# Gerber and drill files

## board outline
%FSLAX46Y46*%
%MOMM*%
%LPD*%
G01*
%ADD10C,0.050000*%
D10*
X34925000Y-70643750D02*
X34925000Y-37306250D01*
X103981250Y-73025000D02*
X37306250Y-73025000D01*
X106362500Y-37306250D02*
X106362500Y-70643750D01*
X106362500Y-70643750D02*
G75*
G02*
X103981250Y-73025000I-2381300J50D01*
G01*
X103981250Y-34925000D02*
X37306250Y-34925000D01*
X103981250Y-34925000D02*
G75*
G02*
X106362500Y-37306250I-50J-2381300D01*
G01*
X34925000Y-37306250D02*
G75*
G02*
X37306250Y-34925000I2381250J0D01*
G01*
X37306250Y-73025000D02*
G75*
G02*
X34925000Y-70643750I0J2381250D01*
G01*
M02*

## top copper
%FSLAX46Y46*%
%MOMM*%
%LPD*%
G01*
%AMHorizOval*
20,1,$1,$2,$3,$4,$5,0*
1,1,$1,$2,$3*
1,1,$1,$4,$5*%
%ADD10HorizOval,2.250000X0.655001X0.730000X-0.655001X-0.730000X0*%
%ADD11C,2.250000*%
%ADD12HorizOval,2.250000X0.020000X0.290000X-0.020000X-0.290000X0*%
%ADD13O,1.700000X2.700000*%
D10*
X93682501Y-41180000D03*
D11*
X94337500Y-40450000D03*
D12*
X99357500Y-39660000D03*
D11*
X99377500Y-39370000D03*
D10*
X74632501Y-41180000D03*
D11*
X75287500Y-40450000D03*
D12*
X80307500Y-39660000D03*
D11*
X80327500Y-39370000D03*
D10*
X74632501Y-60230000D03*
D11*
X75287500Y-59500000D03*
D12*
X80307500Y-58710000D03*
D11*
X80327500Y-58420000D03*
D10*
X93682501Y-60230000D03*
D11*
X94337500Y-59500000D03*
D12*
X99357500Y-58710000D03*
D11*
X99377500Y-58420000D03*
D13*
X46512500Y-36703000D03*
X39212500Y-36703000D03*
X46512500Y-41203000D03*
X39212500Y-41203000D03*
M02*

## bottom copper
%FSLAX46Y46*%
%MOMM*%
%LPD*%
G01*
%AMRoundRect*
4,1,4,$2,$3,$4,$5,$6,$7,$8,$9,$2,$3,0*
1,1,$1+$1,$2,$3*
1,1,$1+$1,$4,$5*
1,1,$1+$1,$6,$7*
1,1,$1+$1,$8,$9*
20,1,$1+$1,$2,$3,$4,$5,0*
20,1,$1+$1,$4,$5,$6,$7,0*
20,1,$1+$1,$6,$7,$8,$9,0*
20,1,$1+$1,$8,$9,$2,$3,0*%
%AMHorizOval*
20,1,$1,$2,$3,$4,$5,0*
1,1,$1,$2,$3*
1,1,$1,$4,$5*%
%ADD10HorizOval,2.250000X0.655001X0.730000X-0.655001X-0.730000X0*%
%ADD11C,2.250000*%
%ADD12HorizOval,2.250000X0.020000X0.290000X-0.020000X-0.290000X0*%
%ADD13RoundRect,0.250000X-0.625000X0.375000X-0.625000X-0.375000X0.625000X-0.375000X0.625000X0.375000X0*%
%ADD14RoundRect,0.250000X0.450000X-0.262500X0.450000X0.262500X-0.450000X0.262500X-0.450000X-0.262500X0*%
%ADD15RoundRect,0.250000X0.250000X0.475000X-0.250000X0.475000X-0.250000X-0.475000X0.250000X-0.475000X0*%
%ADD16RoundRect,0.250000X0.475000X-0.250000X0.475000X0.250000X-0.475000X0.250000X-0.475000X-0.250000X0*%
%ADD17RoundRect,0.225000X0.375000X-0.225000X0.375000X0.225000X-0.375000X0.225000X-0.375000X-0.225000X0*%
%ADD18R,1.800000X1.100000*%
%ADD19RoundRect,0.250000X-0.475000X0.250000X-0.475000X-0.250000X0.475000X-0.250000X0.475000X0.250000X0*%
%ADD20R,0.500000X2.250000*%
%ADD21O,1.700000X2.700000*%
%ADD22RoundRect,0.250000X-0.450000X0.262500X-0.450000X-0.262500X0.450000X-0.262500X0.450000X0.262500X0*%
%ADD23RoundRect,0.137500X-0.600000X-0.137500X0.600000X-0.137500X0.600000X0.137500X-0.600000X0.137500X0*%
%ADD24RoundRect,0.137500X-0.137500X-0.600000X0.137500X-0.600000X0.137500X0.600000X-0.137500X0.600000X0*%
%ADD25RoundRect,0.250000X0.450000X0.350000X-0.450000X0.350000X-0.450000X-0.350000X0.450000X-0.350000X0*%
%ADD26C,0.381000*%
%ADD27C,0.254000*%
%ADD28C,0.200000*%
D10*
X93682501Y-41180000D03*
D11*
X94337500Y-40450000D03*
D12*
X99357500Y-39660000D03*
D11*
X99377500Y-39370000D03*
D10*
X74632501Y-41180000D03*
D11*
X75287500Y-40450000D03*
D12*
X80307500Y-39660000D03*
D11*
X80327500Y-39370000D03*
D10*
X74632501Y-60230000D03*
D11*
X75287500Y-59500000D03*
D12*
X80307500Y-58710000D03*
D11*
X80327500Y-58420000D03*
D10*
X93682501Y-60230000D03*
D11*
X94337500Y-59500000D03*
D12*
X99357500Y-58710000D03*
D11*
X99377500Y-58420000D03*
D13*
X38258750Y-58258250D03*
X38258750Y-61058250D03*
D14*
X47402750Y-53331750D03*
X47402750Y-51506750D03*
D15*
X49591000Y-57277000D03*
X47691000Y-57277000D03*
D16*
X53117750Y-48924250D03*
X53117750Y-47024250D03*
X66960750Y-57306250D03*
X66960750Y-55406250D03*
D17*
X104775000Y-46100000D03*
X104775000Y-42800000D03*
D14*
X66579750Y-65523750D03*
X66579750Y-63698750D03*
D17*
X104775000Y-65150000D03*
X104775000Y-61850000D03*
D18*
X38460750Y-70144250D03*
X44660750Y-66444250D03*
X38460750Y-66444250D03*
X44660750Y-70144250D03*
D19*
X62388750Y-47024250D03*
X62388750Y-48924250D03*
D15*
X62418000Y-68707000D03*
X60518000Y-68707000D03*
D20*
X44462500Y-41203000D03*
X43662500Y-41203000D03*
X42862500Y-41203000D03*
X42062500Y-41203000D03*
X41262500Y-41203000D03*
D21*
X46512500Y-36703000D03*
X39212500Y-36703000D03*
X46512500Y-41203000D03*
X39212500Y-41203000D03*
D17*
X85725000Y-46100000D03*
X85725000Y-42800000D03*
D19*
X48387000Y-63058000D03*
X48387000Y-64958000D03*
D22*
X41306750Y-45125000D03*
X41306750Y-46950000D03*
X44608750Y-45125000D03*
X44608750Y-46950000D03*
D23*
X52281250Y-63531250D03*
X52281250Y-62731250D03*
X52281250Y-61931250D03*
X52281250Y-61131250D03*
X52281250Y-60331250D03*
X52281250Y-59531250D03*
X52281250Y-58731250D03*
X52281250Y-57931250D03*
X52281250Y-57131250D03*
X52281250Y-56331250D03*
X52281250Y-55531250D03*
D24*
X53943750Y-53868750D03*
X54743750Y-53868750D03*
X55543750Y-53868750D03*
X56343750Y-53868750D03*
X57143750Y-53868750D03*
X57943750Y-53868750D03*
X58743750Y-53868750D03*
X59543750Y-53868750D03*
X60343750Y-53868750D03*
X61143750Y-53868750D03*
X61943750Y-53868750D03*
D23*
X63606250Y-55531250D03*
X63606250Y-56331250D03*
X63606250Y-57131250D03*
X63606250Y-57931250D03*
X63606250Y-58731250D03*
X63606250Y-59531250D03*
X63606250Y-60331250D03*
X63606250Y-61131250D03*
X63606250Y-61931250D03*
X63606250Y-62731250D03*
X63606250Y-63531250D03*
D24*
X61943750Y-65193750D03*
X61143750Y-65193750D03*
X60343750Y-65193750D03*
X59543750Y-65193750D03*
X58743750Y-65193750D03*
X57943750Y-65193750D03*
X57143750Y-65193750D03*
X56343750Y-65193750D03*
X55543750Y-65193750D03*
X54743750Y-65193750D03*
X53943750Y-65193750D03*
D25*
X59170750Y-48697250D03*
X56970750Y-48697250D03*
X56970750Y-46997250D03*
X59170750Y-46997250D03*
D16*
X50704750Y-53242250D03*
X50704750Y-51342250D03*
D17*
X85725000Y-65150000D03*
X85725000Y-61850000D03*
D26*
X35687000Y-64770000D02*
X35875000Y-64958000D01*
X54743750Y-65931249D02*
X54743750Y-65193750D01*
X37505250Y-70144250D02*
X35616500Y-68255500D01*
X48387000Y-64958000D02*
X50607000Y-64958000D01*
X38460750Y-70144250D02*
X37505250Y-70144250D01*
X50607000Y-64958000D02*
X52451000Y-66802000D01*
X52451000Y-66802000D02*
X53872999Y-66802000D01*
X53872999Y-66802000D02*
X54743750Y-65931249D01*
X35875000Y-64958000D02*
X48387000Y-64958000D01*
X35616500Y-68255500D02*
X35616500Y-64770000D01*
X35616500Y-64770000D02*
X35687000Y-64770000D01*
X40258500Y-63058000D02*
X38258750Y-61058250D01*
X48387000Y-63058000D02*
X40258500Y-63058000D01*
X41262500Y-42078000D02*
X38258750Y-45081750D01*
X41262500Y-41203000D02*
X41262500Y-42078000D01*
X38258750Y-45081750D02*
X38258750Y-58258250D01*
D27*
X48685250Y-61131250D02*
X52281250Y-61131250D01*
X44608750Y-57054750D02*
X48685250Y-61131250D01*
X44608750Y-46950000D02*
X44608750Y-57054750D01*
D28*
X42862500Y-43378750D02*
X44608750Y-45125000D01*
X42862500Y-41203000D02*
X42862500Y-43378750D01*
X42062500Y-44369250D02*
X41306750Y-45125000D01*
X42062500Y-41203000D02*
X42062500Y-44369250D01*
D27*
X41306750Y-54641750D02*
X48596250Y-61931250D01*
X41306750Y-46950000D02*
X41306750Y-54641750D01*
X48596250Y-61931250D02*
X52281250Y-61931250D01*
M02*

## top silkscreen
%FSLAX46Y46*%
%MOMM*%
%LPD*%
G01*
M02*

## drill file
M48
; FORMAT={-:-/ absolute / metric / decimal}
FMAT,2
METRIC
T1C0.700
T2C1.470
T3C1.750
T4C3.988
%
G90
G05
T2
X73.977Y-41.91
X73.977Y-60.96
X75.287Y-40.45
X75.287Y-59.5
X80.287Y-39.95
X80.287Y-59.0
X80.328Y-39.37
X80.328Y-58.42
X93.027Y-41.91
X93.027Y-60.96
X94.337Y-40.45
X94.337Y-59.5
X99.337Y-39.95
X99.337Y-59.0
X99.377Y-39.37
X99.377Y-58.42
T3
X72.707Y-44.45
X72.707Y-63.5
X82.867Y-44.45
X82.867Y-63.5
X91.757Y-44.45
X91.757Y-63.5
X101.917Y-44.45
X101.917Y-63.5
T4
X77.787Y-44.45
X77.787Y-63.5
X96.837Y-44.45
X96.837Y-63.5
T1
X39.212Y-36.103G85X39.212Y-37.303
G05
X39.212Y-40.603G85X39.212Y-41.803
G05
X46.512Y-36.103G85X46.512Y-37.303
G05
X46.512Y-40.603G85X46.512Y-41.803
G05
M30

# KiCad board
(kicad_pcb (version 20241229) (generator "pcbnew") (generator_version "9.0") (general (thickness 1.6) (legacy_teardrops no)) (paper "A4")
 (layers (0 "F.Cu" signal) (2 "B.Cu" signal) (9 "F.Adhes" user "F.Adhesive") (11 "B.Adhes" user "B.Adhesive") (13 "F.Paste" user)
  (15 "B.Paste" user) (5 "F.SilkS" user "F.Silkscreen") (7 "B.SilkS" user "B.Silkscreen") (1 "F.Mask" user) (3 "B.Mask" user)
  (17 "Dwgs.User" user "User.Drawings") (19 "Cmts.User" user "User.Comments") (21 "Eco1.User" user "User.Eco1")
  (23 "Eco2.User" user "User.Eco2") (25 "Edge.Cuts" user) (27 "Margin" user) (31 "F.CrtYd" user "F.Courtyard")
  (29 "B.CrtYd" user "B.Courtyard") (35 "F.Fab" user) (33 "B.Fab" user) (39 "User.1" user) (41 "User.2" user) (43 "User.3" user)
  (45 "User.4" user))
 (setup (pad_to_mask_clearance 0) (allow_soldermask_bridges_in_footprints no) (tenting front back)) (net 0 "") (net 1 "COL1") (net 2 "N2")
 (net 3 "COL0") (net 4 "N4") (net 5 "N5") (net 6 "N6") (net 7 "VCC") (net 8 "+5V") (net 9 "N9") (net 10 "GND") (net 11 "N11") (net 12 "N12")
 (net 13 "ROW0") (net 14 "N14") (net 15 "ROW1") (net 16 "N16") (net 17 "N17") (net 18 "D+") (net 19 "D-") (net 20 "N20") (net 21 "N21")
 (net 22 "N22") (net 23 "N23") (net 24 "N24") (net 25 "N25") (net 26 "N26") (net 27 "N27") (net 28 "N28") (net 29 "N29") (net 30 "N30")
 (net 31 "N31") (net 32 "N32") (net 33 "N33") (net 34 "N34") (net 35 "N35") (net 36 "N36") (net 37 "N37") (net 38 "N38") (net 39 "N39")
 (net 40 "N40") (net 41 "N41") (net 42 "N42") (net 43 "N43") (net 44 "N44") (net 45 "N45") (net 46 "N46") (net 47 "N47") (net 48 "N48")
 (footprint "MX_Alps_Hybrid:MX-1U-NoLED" (layer "F.Cu") (at 96.8375 44.45)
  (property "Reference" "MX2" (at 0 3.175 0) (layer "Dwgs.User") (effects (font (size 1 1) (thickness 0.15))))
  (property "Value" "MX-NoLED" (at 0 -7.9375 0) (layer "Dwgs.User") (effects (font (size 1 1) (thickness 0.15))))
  (pad "" np_thru_hole circle (at -5.08 0 48.0996) (size 1.75 1.75) (drill 1.75) (layers "*.Cu" "*.Mask"))
  (pad "" np_thru_hole circle (at 0 0) (size 3.9878 3.9878) (drill 3.9878) (layers "*.Cu" "*.Mask"))
  (pad "" np_thru_hole circle (at 5.08 0 48.0996) (size 1.75 1.75) (drill 1.75) (layers "*.Cu" "*.Mask"))
  (pad "1" thru_hole oval (at -3.81 -2.54 48.0996) (size 4.211556 2.25) (drill 1.47 (offset 0.980778 0)) (layers "*.Cu" "B.Mask")
   (remove_unused_layers no) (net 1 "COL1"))
  (pad "1" thru_hole circle (at -2.5 -4) (size 2.25 2.25) (drill 1.47) (layers "*.Cu" "B.Mask") (remove_unused_layers no) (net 1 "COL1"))
  (pad "2" thru_hole oval (at 2.5 -4.5 86.0548) (size 2.831378 2.25) (drill 1.47 (offset 0.290689 0)) (layers "*.Cu" "B.Mask")
   (remove_unused_layers no) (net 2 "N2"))
  (pad "2" thru_hole circle (at 2.54 -5.08) (size 2.25 2.25) (drill 1.47) (layers "*.Cu" "B.Mask") (remove_unused_layers no) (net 2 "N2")))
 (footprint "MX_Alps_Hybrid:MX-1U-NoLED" (layer "F.Cu") (at 77.7875 44.45)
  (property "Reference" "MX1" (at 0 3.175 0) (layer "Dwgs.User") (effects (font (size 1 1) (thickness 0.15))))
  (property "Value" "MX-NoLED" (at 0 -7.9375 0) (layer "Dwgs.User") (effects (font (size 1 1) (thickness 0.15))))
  (pad "" np_thru_hole circle (at -5.08 0 48.0996) (size 1.75 1.75) (drill 1.75) (layers "*.Cu" "*.Mask"))
  (pad "" np_thru_hole circle (at 0 0) (size 3.9878 3.9878) (drill 3.9878) (layers "*.Cu" "*.Mask"))
  (pad "" np_thru_hole circle (at 5.08 0 48.0996) (size 1.75 1.75) (drill 1.75) (layers "*.Cu" "*.Mask"))
  (pad "1" thru_hole oval (at -3.81 -2.54 48.0996) (size 4.211556 2.25) (drill 1.47 (offset 0.980778 0)) (layers "*.Cu" "B.Mask")
   (remove_unused_layers no) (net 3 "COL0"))
  (pad "1" thru_hole circle (at -2.5 -4) (size 2.25 2.25) (drill 1.47) (layers "*.Cu" "B.Mask") (remove_unused_layers no) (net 3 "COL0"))
  (pad "2" thru_hole oval (at 2.5 -4.5 86.0548) (size 2.831378 2.25) (drill 1.47 (offset 0.290689 0)) (layers "*.Cu" "B.Mask")
   (remove_unused_layers no) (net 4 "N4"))
  (pad "2" thru_hole circle (at 2.54 -5.08) (size 2.25 2.25) (drill 1.47) (layers "*.Cu" "B.Mask") (remove_unused_layers no) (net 4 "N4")))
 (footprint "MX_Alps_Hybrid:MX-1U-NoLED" (layer "F.Cu") (at 77.7875 63.5)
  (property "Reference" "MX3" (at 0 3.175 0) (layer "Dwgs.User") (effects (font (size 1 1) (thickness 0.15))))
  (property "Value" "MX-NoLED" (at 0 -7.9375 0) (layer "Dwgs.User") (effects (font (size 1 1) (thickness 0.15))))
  (pad "" np_thru_hole circle (at -5.08 0 48.0996) (size 1.75 1.75) (drill 1.75) (layers "*.Cu" "*.Mask"))
  (pad "" np_thru_hole circle (at 0 0) (size 3.9878 3.9878) (drill 3.9878) (layers "*.Cu" "*.Mask"))
  (pad "" np_thru_hole circle (at 5.08 0 48.0996) (size 1.75 1.75) (drill 1.75) (layers "*.Cu" "*.Mask"))
  (pad "1" thru_hole oval (at -3.81 -2.54 48.0996) (size 4.211556 2.25) (drill 1.47 (offset 0.980778 0)) (layers "*.Cu" "B.Mask")
   (remove_unused_layers no) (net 3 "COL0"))
  (pad "1" thru_hole circle (at -2.5 -4) (size 2.25 2.25) (drill 1.47) (layers "*.Cu" "B.Mask") (remove_unused_layers no) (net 3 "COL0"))
  (pad "2" thru_hole oval (at 2.5 -4.5 86.0548) (size 2.831378 2.25) (drill 1.47 (offset 0.290689 0)) (layers "*.Cu" "B.Mask")
   (remove_unused_layers no) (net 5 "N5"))
  (pad "2" thru_hole circle (at 2.54 -5.08) (size 2.25 2.25) (drill 1.47) (layers "*.Cu" "B.Mask") (remove_unused_layers no) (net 5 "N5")))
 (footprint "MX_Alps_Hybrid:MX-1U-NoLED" (layer "F.Cu") (at 96.8375 63.5)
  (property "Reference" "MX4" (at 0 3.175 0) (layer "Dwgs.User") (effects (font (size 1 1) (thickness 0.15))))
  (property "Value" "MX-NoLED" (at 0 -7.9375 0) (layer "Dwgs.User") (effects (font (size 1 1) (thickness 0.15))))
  (pad "" np_thru_hole circle (at -5.08 0 48.0996) (size 1.75 1.75) (drill 1.75) (layers "*.Cu" "*.Mask"))
  (pad "" np_thru_hole circle (at 0 0) (size 3.9878 3.9878) (drill 3.9878) (layers "*.Cu" "*.Mask"))
  (pad "" np_thru_hole circle (at 5.08 0 48.0996) (size 1.75 1.75) (drill 1.75) (layers "*.Cu" "*.Mask"))
  (pad "1" thru_hole oval (at -3.81 -2.54 48.0996) (size 4.211556 2.25) (drill 1.47 (offset 0.980778 0)) (layers "*.Cu" "B.Mask")
   (remove_unused_layers no) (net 1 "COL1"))
  (pad "1" thru_hole circle (at -2.5 -4) (size 2.25 2.25) (drill 1.47) (layers "*.Cu" "B.Mask") (remove_unused_layers no) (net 1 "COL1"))
  (pad "2" thru_hole oval (at 2.5 -4.5 86.0548) (size 2.831378 2.25) (drill 1.47 (offset 0.290689 0)) (layers "*.Cu" "B.Mask")
   (remove_unused_layers no) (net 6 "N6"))
  (pad "2" thru_hole circle (at 2.54 -5.08) (size 2.25 2.25) (drill 1.47) (layers "*.Cu" "B.Mask") (remove_unused_layers no) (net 6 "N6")))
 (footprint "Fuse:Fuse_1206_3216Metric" (layer "B.Cu") (at 38.25875 59.65825 -90)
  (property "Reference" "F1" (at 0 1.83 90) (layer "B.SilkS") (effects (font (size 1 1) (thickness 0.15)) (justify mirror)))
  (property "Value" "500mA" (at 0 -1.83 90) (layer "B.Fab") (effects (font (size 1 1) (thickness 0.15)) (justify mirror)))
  (pad "1" smd roundrect (at -1.4 0 270) (size 1.25 1.75) (layers "B.Cu" "B.Mask" "B.Paste") (roundrect_rratio 0.2) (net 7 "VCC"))
  (pad "2" smd roundrect (at 1.4 0 270) (size 1.25 1.75) (layers "B.Cu" "B.Mask" "B.Paste") (roundrect_rratio 0.2) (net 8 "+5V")))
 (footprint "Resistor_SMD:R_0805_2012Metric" (layer "B.Cu") (at 47.40275 52.41925 90)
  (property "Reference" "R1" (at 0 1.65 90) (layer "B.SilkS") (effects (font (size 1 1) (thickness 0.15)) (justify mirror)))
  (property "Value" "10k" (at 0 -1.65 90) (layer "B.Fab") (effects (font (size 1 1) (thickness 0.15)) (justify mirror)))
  (pad "1" smd roundrect (at -0.9125 0 90) (size 1.025 1.4) (layers "B.Cu" "B.Mask" "B.Paste") (roundrect_rratio 0.243902) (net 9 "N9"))
  (pad "2" smd roundrect (at 0.9125 0 90) (size 1.025 1.4) (layers "B.Cu" "B.Mask" "B.Paste") (roundrect_rratio 0.243902) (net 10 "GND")))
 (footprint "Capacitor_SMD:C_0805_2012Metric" (layer "B.Cu") (at 48.641 57.277 180)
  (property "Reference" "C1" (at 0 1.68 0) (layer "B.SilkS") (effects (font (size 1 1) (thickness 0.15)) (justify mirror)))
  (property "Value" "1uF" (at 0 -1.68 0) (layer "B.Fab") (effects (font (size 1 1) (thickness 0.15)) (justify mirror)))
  (pad "1" smd roundrect (at -0.95 0 180) (size 1 1.45) (layers "B.Cu" "B.Mask" "B.Paste") (roundrect_rratio 0.25) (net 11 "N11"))
  (pad "2" smd roundrect (at 0.95 0 180) (size 1 1.45) (layers "B.Cu" "B.Mask" "B.Paste") (roundrect_rratio 0.25) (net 10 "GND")))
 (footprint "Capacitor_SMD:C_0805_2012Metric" (layer "B.Cu") (at 53.11775 47.97425 90)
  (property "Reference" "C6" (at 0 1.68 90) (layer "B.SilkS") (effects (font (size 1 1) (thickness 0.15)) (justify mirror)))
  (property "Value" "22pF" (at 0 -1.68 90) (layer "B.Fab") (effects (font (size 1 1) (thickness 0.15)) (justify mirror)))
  (pad "1" smd roundrect (at -0.95 0 90) (size 1 1.45) (layers "B.Cu" "B.Mask" "B.Paste") (roundrect_rratio 0.25) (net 10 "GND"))
  (pad "2" smd roundrect (at 0.95 0 90) (size 1 1.45) (layers "B.Cu" "B.Mask" "B.Paste") (roundrect_rratio 0.25) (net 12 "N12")))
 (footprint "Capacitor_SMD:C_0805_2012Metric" (layer "B.Cu") (at 66.96075 56.35625 90)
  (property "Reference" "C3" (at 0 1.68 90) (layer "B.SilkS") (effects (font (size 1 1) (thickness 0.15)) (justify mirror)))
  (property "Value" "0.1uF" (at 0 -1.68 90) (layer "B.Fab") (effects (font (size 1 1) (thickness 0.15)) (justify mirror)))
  (pad "1" smd roundrect (at -0.95 0 90) (size 1 1.45) (layers "B.Cu" "B.Mask" "B.Paste") (roundrect_rratio 0.25) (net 8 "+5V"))
  (pad "2" smd roundrect (at 0.95 0 90) (size 1 1.45) (layers "B.Cu" "B.Mask" "B.Paste") (roundrect_rratio 0.25) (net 10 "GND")))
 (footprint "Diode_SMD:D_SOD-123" (layer "B.Cu") (at 104.775 44.45 90)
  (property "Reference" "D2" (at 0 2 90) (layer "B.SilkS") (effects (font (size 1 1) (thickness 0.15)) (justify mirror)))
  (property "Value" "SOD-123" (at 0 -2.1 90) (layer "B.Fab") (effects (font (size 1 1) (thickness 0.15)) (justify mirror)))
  (pad "1" smd roundrect (at -1.65 0 90) (size 0.9 1.2) (layers "B.Cu" "B.Mask" "B.Paste") (roundrect_rratio 0.25) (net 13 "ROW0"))
  (pad "2" smd roundrect (at 1.65 0 90) (size 0.9 1.2) (layers "B.Cu" "B.Mask" "B.Paste") (roundrect_rratio 0.25) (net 2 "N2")))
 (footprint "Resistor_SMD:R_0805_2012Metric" (layer "B.Cu") (at 66.57975 64.61125 90)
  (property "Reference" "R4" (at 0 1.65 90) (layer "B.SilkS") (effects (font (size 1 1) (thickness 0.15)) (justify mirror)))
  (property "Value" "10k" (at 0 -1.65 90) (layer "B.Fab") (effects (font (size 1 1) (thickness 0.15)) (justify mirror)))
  (pad "1" smd roundrect (at -0.9125 0 90) (size 1.025 1.4) (layers "B.Cu" "B.Mask" "B.Paste") (roundrect_rratio 0.243902) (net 8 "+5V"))
  (pad "2" smd roundrect (at 0.9125 0 90) (size 1.025 1.4) (layers "B.Cu" "B.Mask" "B.Paste") (roundrect_rratio 0.243902) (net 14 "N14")))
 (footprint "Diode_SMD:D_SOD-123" (layer "B.Cu") (at 104.775 63.5 90)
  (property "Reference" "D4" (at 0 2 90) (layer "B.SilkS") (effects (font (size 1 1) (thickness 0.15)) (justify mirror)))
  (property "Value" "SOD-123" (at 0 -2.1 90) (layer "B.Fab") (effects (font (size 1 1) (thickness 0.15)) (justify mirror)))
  (pad "1" smd roundrect (at -1.65 0 90) (size 0.9 1.2) (layers "B.Cu" "B.Mask" "B.Paste") (roundrect_rratio 0.25) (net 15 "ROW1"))
  (pad "2" smd roundrect (at 1.65 0 90) (size 0.9 1.2) (layers "B.Cu" "B.Mask" "B.Paste") (roundrect_rratio 0.25) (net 6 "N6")))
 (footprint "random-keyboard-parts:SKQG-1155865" (layer "B.Cu") (at 41.56075 68.29425 180)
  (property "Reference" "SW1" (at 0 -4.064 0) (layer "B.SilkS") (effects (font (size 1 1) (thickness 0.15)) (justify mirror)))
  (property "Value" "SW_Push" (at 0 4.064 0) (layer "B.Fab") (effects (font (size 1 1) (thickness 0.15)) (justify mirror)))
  (pad "1" smd rect (at 3.1 -1.85 180) (size 1.8 1.1) (layers "B.Cu" "B.Mask" "B.Paste") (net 10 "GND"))
  (pad "2" smd rect (at -3.1 1.85 180) (size 1.8 1.1) (layers "B.Cu" "B.Mask" "B.Paste") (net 14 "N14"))
  (pad "3" smd rect (at 3.1 1.85 180) (size 1.8 1.1) (layers "B.Cu" "B.Mask" "B.Paste"))
  (pad "4" smd rect (at -3.1 -1.85 180) (size 1.8 1.1) (layers "B.Cu" "B.Mask" "B.Paste")))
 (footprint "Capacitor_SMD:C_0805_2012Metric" (layer "B.Cu") (at 62.38875 47.97425 -90)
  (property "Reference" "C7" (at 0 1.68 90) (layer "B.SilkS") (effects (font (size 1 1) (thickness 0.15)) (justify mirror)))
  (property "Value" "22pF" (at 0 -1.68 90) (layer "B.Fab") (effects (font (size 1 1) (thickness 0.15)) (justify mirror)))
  (pad "1" smd roundrect (at -0.95 0 270) (size 1 1.45) (layers "B.Cu" "B.Mask" "B.Paste") (roundrect_rratio 0.25) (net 10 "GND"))
  (pad "2" smd roundrect (at 0.95 0 270) (size 1 1.45) (layers "B.Cu" "B.Mask" "B.Paste") (roundrect_rratio 0.25) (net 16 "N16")))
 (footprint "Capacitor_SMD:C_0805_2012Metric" (layer "B.Cu") (at 61.468 68.707 180)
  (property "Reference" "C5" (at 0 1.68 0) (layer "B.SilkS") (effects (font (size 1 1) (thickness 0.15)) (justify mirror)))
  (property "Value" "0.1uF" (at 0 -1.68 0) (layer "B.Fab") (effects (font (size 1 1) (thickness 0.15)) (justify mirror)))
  (pad "1" smd roundrect (at -0.95 0 180) (size 1 1.45) (layers "B.Cu" "B.Mask" "B.Paste") (roundrect_rratio 0.25) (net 8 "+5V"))
  (pad "2" smd roundrect (at 0.95 0 180) (size 1 1.45) (layers "B.Cu" "B.Mask" "B.Paste") (roundrect_rratio 0.25) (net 10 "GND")))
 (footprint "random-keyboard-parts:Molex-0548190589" (layer "B.Cu") (at 42.8625 36.703 -90)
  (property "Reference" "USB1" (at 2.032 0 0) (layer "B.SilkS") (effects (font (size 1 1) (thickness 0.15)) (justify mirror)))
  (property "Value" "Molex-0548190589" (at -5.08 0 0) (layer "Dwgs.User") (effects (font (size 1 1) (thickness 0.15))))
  (pad "1" smd rect (at 4.5 -1.6 270) (size 2.25 0.5) (layers "B.Cu" "B.Mask" "B.Paste") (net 10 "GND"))
  (pad "2" smd rect (at 4.5 -0.8 270) (size 2.25 0.5) (layers "B.Cu" "B.Mask" "B.Paste") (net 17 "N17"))
  (pad "3" smd rect (at 4.5 0 270) (size 2.25 0.5) (layers "B.Cu" "B.Mask" "B.Paste") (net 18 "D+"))
  (pad "4" smd rect (at 4.5 0.8 270) (size 2.25 0.5) (layers "B.Cu" "B.Mask" "B.Paste") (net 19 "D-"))
  (pad "5" smd rect (at 4.5 1.6 270) (size 2.25 0.5) (layers "B.Cu" "B.Mask" "B.Paste") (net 7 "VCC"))
  (pad "6" thru_hole oval (at 0 -3.65 270) (size 2.7 1.7) (drill oval 1.9 0.7) (layers "*.Cu" "*.Mask") (remove_unused_layers no)
   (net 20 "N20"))
  (pad "6" thru_hole oval (at 0 3.65 270) (size 2.7 1.7) (drill oval 1.9 0.7) (layers "*.Cu" "*.Mask") (remove_unused_layers no)
   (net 20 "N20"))
  (pad "6" thru_hole oval (at 4.5 -3.65 270) (size 2.7 1.7) (drill oval 1.9 0.7) (layers "*.Cu" "*.Mask") (remove_unused_layers no)
   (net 20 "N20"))
  (pad "6" thru_hole oval (at 4.5 3.65 270) (size 2.7 1.7) (drill oval 1.9 0.7) (layers "*.Cu" "*.Mask") (remove_unused_layers no)
   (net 20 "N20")))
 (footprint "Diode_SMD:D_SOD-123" (layer "B.Cu") (at 85.725 44.45 90)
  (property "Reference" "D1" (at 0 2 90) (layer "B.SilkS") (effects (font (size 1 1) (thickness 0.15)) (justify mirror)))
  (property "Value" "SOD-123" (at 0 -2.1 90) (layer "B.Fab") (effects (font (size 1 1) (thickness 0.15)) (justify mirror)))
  (pad "1" smd roundrect (at -1.65 0 90) (size 0.9 1.2) (layers "B.Cu" "B.Mask" "B.Paste") (roundrect_rratio 0.25) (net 13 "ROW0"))
  (pad "2" smd roundrect (at 1.65 0 90) (size 0.9 1.2) (layers "B.Cu" "B.Mask" "B.Paste") (roundrect_rratio 0.25) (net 4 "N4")))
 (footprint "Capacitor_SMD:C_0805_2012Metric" (layer "B.Cu") (at 48.387 64.008 -90)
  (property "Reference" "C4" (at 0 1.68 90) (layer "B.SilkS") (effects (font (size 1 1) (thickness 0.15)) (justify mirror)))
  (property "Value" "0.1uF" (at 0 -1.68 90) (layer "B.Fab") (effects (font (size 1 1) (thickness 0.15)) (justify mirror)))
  (pad "1" smd roundrect (at -0.95 0 270) (size 1 1.45) (layers "B.Cu" "B.Mask" "B.Paste") (roundrect_rratio 0.25) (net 8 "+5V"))
  (pad "2" smd roundrect (at 0.95 0 270) (size 1 1.45) (layers "B.Cu" "B.Mask" "B.Paste") (roundrect_rratio 0.25) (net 10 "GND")))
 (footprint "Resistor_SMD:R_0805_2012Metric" (layer "B.Cu") (at 41.30675 46.0375 -90)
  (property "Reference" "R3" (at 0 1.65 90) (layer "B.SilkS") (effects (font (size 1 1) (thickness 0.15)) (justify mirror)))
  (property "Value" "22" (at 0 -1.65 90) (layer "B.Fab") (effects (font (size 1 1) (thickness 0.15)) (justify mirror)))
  (pad "1" smd roundrect (at -0.9125 0 270) (size 1.025 1.4) (layers "B.Cu" "B.Mask" "B.Paste") (roundrect_rratio 0.243902) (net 19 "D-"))
  (pad "2" smd roundrect (at 0.9125 0 270) (size 1.025 1.4) (layers "B.Cu" "B.Mask" "B.Paste") (roundrect_rratio 0.243902) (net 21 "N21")))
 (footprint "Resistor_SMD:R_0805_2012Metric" (layer "B.Cu") (at 44.60875 46.0375 -90)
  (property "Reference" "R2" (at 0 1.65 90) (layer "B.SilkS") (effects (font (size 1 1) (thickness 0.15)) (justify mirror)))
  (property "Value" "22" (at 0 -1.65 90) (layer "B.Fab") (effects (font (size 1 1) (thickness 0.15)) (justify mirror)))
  (pad "1" smd roundrect (at -0.9125 0 270) (size 1.025 1.4) (layers "B.Cu" "B.Mask" "B.Paste") (roundrect_rratio 0.243902) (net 18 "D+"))
  (pad "2" smd roundrect (at 0.9125 0 270) (size 1.025 1.4) (layers "B.Cu" "B.Mask" "B.Paste") (roundrect_rratio 0.243902) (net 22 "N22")))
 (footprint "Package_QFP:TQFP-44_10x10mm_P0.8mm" (layer "B.Cu") (at 57.94375 59.53125)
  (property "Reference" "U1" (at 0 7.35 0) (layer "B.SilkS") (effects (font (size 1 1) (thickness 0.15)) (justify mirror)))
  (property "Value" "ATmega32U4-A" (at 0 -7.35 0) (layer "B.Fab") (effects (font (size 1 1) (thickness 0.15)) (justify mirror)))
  (pad "1" smd roundrect (at -5.6625 4) (size 1.475 0.55) (layers "B.Cu" "B.Mask" "B.Paste") (roundrect_rratio 0.25) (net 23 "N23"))
  (pad "2" smd roundrect (at -5.6625 3.2) (size 1.475 0.55) (layers "B.Cu" "B.Mask" "B.Paste") (roundrect_rratio 0.25) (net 8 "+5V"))
  (pad "3" smd roundrect (at -5.6625 2.4) (size 1.475 0.55) (layers "B.Cu" "B.Mask" "B.Paste") (roundrect_rratio 0.25) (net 21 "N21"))
  (pad "4" smd roundrect (at -5.6625 1.6) (size 1.475 0.55) (layers "B.Cu" "B.Mask" "B.Paste") (roundrect_rratio 0.25) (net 22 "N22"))
  (pad "5" smd roundrect (at -5.6625 0.8) (size 1.475 0.55) (layers "B.Cu" "B.Mask" "B.Paste") (roundrect_rratio 0.25) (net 10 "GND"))
  (pad "6" smd roundrect (at -5.6625 0) (size 1.475 0.55) (layers "B.Cu" "B.Mask" "B.Paste") (roundrect_rratio 0.25) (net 11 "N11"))
  (pad "7" smd roundrect (at -5.6625 -0.8) (size 1.475 0.55) (layers "B.Cu" "B.Mask" "B.Paste") (roundrect_rratio 0.25) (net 8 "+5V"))
  (pad "8" smd roundrect (at -5.6625 -1.6) (size 1.475 0.55) (layers "B.Cu" "B.Mask" "B.Paste") (roundrect_rratio 0.25) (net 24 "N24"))
  (pad "9" smd roundrect (at -5.6625 -2.4) (size 1.475 0.55) (layers "B.Cu" "B.Mask" "B.Paste") (roundrect_rratio 0.25) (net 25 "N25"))
  (pad "10" smd roundrect (at -5.6625 -3.2) (size 1.475 0.55) (layers "B.Cu" "B.Mask" "B.Paste") (roundrect_rratio 0.25) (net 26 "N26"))
  (pad "11" smd roundrect (at -5.6625 -4) (size 1.475 0.55) (layers "B.Cu" "B.Mask" "B.Paste") (roundrect_rratio 0.25) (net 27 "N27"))
  (pad "12" smd roundrect (at -4 -5.6625) (size 0.55 1.475) (layers "B.Cu" "B.Mask" "B.Paste") (roundrect_rratio 0.25) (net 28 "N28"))
  (pad "13" smd roundrect (at -3.2 -5.6625) (size 0.55 1.475) (layers "B.Cu" "B.Mask" "B.Paste") (roundrect_rratio 0.25) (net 14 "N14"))
  (pad "14" smd roundrect (at -2.4 -5.6625) (size 0.55 1.475) (layers "B.Cu" "B.Mask" "B.Paste") (roundrect_rratio 0.25) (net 8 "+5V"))
  (pad "15" smd roundrect (at -1.6 -5.6625) (size 0.55 1.475) (layers "B.Cu" "B.Mask" "B.Paste") (roundrect_rratio 0.25) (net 10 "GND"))
  (pad "16" smd roundrect (at -0.8 -5.6625) (size 0.55 1.475) (layers "B.Cu" "B.Mask" "B.Paste") (roundrect_rratio 0.25) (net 16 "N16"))
  (pad "17" smd roundrect (at 0 -5.6625) (size 0.55 1.475) (layers "B.Cu" "B.Mask" "B.Paste") (roundrect_rratio 0.25) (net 12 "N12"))
  (pad "18" smd roundrect (at 0.8 -5.6625) (size 0.55 1.475) (layers "B.Cu" "B.Mask" "B.Paste") (roundrect_rratio 0.25) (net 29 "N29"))
  (pad "19" smd roundrect (at 1.6 -5.6625) (size 0.55 1.475) (layers "B.Cu" "B.Mask" "B.Paste") (roundrect_rratio 0.25) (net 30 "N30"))
  (pad "20" smd roundrect (at 2.4 -5.6625) (size 0.55 1.475) (layers "B.Cu" "B.Mask" "B.Paste") (roundrect_rratio 0.25) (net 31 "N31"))
  (pad "21" smd roundrect (at 3.2 -5.6625) (size 0.55 1.475) (layers "B.Cu" "B.Mask" "B.Paste") (roundrect_rratio 0.25) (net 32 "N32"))
  (pad "22" smd roundrect (at 4 -5.6625) (size 0.55 1.475) (layers "B.Cu" "B.Mask" "B.Paste") (roundrect_rratio 0.25) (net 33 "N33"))
  (pad "23" smd roundrect (at 5.6625 -4) (size 1.475 0.55) (layers "B.Cu" "B.Mask" "B.Paste") (roundrect_rratio 0.25) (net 10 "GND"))
  (pad "24" smd roundrect (at 5.6625 -3.2) (size 1.475 0.55) (layers "B.Cu" "B.Mask" "B.Paste") (roundrect_rratio 0.25) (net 8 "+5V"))
  (pad "25" smd roundrect (at 5.6625 -2.4) (size 1.475 0.55) (layers "B.Cu" "B.Mask" "B.Paste") (roundrect_rratio 0.25) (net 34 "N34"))
  (pad "26" smd roundrect (at 5.6625 -1.6) (size 1.475 0.55) (layers "B.Cu" "B.Mask" "B.Paste") (roundrect_rratio 0.25) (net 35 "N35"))
  (pad "27" smd roundrect (at 5.6625 -0.8) (size 1.475 0.55) (layers "B.Cu" "B.Mask" "B.Paste") (roundrect_rratio 0.25) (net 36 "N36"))
  (pad "28" smd roundrect (at 5.6625 0) (size 1.475 0.55) (layers "B.Cu" "B.Mask" "B.Paste") (roundrect_rratio 0.25) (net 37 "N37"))
  (pad "29" smd roundrect (at 5.6625 0.8) (size 1.475 0.55) (layers "B.Cu" "B.Mask" "B.Paste") (roundrect_rratio 0.25) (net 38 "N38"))
  (pad "30" smd roundrect (at 5.6625 1.6) (size 1.475 0.55) (layers "B.Cu" "B.Mask" "B.Paste") (roundrect_rratio 0.25) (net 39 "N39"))
  (pad "31" smd roundrect (at 5.6625 2.4) (size 1.475 0.55) (layers "B.Cu" "B.Mask" "B.Paste") (roundrect_rratio 0.25) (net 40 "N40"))
  (pad "32" smd roundrect (at 5.6625 3.2) (size 1.475 0.55) (layers "B.Cu" "B.Mask" "B.Paste") (roundrect_rratio 0.25) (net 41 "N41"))
  (pad "33" smd roundrect (at 5.6625 4) (size 1.475 0.55) (layers "B.Cu" "B.Mask" "B.Paste") (roundrect_rratio 0.25) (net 9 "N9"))
  (pad "34" smd roundrect (at 4 5.6625) (size 0.55 1.475) (layers "B.Cu" "B.Mask" "B.Paste") (roundrect_rratio 0.25) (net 8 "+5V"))
  (pad "35" smd roundrect (at 3.2 5.6625) (size 0.55 1.475) (layers "B.Cu" "B.Mask" "B.Paste") (roundrect_rratio 0.25) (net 10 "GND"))
  (pad "36" smd roundrect (at 2.4 5.6625) (size 0.55 1.475) (layers "B.Cu" "B.Mask" "B.Paste") (roundrect_rratio 0.25) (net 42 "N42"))
  (pad "37" smd roundrect (at 1.6 5.6625) (size 0.55 1.475) (layers "B.Cu" "B.Mask" "B.Paste") (roundrect_rratio 0.25) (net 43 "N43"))
  (pad "38" smd roundrect (at 0.8 5.6625) (size 0.55 1.475) (layers "B.Cu" "B.Mask" "B.Paste") (roundrect_rratio 0.25) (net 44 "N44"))
  (pad "39" smd roundrect (at 0 5.6625) (size 0.55 1.475) (layers "B.Cu" "B.Mask" "B.Paste") (roundrect_rratio 0.25) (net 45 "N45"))
  (pad "40" smd roundrect (at -0.8 5.6625) (size 0.55 1.475) (layers "B.Cu" "B.Mask" "B.Paste") (roundrect_rratio 0.25) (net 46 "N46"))
  (pad "41" smd roundrect (at -1.6 5.6625) (size 0.55 1.475) (layers "B.Cu" "B.Mask" "B.Paste") (roundrect_rratio 0.25) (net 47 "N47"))
  (pad "42" smd roundrect (at -2.4 5.6625) (size 0.55 1.475) (layers "B.Cu" "B.Mask" "B.Paste") (roundrect_rratio 0.25) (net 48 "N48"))
  (pad "43" smd roundrect (at -3.2 5.6625) (size 0.55 1.475) (layers "B.Cu" "B.Mask" "B.Paste") (roundrect_rratio 0.25) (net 10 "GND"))
  (pad "44" smd roundrect (at -4 5.6625) (size 0.55 1.475) (layers "B.Cu" "B.Mask" "B.Paste") (roundrect_rratio 0.25) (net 8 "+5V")))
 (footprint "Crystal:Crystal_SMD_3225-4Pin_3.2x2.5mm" (layer "B.Cu") (at 58.07075 47.84725 180)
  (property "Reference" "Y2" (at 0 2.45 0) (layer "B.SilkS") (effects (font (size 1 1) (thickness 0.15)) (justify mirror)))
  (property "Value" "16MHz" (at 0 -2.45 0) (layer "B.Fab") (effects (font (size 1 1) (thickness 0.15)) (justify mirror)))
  (pad "1" smd roundrect (at -1.1 -0.85 180) (size 1.4 1.2) (layers "B.Cu" "B.Mask" "B.Paste") (roundrect_rratio 0.208333) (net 12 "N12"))
  (pad "2" smd roundrect (at 1.1 -0.85 180) (size 1.4 1.2) (layers "B.Cu" "B.Mask" "B.Paste") (roundrect_rratio 0.208333) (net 10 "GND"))
  (pad "3" smd roundrect (at 1.1 0.85 180) (size 1.4 1.2) (layers "B.Cu" "B.Mask" "B.Paste") (roundrect_rratio 0.208333) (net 16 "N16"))
  (pad "4" smd roundrect (at -1.1 0.85 180) (size 1.4 1.2) (layers "B.Cu" "B.Mask" "B.Paste") (roundrect_rratio 0.208333) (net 10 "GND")))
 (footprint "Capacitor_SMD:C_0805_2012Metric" (layer "B.Cu") (at 50.70475 52.29225 90)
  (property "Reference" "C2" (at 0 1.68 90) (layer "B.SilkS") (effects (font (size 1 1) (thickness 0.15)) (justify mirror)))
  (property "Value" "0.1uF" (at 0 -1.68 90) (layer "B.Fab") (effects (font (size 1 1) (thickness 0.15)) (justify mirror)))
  (pad "1" smd roundrect (at -0.95 0 90) (size 1 1.45) (layers "B.Cu" "B.Mask" "B.Paste") (roundrect_rratio 0.25) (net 8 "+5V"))
  (pad "2" smd roundrect (at 0.95 0 90) (size 1 1.45) (layers "B.Cu" "B.Mask" "B.Paste") (roundrect_rratio 0.25) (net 10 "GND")))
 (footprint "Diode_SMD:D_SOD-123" (layer "B.Cu") (at 85.725 63.5 90)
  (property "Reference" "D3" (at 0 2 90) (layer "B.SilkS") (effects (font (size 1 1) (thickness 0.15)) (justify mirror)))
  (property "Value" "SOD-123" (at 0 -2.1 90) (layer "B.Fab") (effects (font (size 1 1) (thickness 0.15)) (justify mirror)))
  (pad "1" smd roundrect (at -1.65 0 90) (size 0.9 1.2) (layers "B.Cu" "B.Mask" "B.Paste") (roundrect_rratio 0.25) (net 15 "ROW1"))
  (pad "2" smd roundrect (at 1.65 0 90) (size 0.9 1.2) (layers "B.Cu" "B.Mask" "B.Paste") (roundrect_rratio 0.25) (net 5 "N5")))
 (gr_line (start 34.925 70.64375) (end 34.925 37.30625) (stroke (width 0.05) (type default)) (layer "Edge.Cuts"))
 (gr_line (start 103.98125 73.025) (end 37.30625 73.025) (stroke (width 0.05) (type default)) (layer "Edge.Cuts"))
 (gr_line (start 106.3625 37.30625) (end 106.3625 70.64375) (stroke (width 0.05) (type default)) (layer "Edge.Cuts"))
 (gr_arc (start 106.3625 70.64375) (mid 105.665048 72.327548) (end 103.98125 73.025) (stroke (width 0.05) (type default))
  (layer "Edge.Cuts"))
 (gr_line (start 103.98125 34.925) (end 37.30625 34.925) (stroke (width 0.05) (type default)) (layer "Edge.Cuts"))
 (gr_arc (start 103.98125 34.925) (mid 105.665048 35.622452) (end 106.3625 37.30625) (stroke (width 0.05) (type default))
  (layer "Edge.Cuts"))
 (gr_arc (start 34.925 37.30625) (mid 35.622452 35.622452) (end 37.30625 34.925) (stroke (width 0.05) (type default)) (layer "Edge.Cuts"))
 (gr_arc (start 37.30625 73.025) (mid 35.622452 72.327548) (end 34.925 70.64375) (stroke (width 0.05) (type default)) (layer "Edge.Cuts"))
 (segment (start 35.687 64.77) (end 35.875 64.958) (width 0.381) (layer "B.Cu") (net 10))
 (segment (start 54.74375 65.931249) (end 54.74375 65.19375) (width 0.381) (layer "B.Cu") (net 10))
 (segment (start 37.50525 70.14425) (end 35.6165 68.2555) (width 0.381) (layer "B.Cu") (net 10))
 (segment (start 48.387 64.958) (end 50.607 64.958) (width 0.381) (layer "B.Cu") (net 10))
 (segment (start 38.46075 70.14425) (end 37.50525 70.14425) (width 0.381) (layer "B.Cu") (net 10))
 (segment (start 50.607 64.958) (end 52.451 66.802) (width 0.381) (layer "B.Cu") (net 10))
 (segment (start 52.451 66.802) (end 53.872999 66.802) (width 0.381) (layer "B.Cu") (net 10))
 (segment (start 53.872999 66.802) (end 54.74375 65.931249) (width 0.381) (layer "B.Cu") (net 10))
 (segment (start 35.875 64.958) (end 48.387 64.958) (width 0.381) (layer "B.Cu") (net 10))
 (segment (start 35.6165 68.2555) (end 35.6165 64.77) (width 0.381) (layer "B.Cu") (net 10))
 (segment (start 35.6165 64.77) (end 35.687 64.77) (width 0.381) (layer "B.Cu") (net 10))
 (segment (start 40.2585 63.058) (end 38.25875 61.05825) (width 0.381) (layer "B.Cu") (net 8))
 (segment (start 48.387 63.058) (end 40.2585 63.058) (width 0.381) (layer "B.Cu") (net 8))
 (segment (start 41.2625 42.078) (end 38.25875 45.08175) (width 0.381) (layer "B.Cu") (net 7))
 (segment (start 41.2625 41.203) (end 41.2625 42.078) (width 0.381) (layer "B.Cu") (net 7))
 (segment (start 38.25875 45.08175) (end 38.25875 58.25825) (width 0.381) (layer "B.Cu") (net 7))
 (segment (start 48.68525 61.13125) (end 52.28125 61.13125) (width 0.254) (layer "B.Cu") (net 22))
 (segment (start 44.60875 57.05475) (end 48.68525 61.13125) (width 0.254) (layer "B.Cu") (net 22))
 (segment (start 44.60875 46.95) (end 44.60875 57.05475) (width 0.254) (layer "B.Cu") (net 22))
 (segment (start 42.8625 43.37875) (end 44.60875 45.125) (width 0.2) (layer "B.Cu") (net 18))
 (segment (start 42.8625 41.203) (end 42.8625 43.37875) (width 0.2) (layer "B.Cu") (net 18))
 (segment (start 42.0625 44.36925) (end 41.30675 45.125) (width 0.2) (layer "B.Cu") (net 19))
 (segment (start 42.0625 41.203) (end 42.0625 44.36925) (width 0.2) (layer "B.Cu") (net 19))
 (segment (start 41.30675 54.64175) (end 48.59625 61.93125) (width 0.254) (layer "B.Cu") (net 21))
 (segment (start 41.30675 46.95) (end 41.30675 54.64175) (width 0.254) (layer "B.Cu") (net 21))
 (segment (start 48.59625 61.93125) (end 52.28125 61.93125) (width 0.254) (layer "B.Cu") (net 21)))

